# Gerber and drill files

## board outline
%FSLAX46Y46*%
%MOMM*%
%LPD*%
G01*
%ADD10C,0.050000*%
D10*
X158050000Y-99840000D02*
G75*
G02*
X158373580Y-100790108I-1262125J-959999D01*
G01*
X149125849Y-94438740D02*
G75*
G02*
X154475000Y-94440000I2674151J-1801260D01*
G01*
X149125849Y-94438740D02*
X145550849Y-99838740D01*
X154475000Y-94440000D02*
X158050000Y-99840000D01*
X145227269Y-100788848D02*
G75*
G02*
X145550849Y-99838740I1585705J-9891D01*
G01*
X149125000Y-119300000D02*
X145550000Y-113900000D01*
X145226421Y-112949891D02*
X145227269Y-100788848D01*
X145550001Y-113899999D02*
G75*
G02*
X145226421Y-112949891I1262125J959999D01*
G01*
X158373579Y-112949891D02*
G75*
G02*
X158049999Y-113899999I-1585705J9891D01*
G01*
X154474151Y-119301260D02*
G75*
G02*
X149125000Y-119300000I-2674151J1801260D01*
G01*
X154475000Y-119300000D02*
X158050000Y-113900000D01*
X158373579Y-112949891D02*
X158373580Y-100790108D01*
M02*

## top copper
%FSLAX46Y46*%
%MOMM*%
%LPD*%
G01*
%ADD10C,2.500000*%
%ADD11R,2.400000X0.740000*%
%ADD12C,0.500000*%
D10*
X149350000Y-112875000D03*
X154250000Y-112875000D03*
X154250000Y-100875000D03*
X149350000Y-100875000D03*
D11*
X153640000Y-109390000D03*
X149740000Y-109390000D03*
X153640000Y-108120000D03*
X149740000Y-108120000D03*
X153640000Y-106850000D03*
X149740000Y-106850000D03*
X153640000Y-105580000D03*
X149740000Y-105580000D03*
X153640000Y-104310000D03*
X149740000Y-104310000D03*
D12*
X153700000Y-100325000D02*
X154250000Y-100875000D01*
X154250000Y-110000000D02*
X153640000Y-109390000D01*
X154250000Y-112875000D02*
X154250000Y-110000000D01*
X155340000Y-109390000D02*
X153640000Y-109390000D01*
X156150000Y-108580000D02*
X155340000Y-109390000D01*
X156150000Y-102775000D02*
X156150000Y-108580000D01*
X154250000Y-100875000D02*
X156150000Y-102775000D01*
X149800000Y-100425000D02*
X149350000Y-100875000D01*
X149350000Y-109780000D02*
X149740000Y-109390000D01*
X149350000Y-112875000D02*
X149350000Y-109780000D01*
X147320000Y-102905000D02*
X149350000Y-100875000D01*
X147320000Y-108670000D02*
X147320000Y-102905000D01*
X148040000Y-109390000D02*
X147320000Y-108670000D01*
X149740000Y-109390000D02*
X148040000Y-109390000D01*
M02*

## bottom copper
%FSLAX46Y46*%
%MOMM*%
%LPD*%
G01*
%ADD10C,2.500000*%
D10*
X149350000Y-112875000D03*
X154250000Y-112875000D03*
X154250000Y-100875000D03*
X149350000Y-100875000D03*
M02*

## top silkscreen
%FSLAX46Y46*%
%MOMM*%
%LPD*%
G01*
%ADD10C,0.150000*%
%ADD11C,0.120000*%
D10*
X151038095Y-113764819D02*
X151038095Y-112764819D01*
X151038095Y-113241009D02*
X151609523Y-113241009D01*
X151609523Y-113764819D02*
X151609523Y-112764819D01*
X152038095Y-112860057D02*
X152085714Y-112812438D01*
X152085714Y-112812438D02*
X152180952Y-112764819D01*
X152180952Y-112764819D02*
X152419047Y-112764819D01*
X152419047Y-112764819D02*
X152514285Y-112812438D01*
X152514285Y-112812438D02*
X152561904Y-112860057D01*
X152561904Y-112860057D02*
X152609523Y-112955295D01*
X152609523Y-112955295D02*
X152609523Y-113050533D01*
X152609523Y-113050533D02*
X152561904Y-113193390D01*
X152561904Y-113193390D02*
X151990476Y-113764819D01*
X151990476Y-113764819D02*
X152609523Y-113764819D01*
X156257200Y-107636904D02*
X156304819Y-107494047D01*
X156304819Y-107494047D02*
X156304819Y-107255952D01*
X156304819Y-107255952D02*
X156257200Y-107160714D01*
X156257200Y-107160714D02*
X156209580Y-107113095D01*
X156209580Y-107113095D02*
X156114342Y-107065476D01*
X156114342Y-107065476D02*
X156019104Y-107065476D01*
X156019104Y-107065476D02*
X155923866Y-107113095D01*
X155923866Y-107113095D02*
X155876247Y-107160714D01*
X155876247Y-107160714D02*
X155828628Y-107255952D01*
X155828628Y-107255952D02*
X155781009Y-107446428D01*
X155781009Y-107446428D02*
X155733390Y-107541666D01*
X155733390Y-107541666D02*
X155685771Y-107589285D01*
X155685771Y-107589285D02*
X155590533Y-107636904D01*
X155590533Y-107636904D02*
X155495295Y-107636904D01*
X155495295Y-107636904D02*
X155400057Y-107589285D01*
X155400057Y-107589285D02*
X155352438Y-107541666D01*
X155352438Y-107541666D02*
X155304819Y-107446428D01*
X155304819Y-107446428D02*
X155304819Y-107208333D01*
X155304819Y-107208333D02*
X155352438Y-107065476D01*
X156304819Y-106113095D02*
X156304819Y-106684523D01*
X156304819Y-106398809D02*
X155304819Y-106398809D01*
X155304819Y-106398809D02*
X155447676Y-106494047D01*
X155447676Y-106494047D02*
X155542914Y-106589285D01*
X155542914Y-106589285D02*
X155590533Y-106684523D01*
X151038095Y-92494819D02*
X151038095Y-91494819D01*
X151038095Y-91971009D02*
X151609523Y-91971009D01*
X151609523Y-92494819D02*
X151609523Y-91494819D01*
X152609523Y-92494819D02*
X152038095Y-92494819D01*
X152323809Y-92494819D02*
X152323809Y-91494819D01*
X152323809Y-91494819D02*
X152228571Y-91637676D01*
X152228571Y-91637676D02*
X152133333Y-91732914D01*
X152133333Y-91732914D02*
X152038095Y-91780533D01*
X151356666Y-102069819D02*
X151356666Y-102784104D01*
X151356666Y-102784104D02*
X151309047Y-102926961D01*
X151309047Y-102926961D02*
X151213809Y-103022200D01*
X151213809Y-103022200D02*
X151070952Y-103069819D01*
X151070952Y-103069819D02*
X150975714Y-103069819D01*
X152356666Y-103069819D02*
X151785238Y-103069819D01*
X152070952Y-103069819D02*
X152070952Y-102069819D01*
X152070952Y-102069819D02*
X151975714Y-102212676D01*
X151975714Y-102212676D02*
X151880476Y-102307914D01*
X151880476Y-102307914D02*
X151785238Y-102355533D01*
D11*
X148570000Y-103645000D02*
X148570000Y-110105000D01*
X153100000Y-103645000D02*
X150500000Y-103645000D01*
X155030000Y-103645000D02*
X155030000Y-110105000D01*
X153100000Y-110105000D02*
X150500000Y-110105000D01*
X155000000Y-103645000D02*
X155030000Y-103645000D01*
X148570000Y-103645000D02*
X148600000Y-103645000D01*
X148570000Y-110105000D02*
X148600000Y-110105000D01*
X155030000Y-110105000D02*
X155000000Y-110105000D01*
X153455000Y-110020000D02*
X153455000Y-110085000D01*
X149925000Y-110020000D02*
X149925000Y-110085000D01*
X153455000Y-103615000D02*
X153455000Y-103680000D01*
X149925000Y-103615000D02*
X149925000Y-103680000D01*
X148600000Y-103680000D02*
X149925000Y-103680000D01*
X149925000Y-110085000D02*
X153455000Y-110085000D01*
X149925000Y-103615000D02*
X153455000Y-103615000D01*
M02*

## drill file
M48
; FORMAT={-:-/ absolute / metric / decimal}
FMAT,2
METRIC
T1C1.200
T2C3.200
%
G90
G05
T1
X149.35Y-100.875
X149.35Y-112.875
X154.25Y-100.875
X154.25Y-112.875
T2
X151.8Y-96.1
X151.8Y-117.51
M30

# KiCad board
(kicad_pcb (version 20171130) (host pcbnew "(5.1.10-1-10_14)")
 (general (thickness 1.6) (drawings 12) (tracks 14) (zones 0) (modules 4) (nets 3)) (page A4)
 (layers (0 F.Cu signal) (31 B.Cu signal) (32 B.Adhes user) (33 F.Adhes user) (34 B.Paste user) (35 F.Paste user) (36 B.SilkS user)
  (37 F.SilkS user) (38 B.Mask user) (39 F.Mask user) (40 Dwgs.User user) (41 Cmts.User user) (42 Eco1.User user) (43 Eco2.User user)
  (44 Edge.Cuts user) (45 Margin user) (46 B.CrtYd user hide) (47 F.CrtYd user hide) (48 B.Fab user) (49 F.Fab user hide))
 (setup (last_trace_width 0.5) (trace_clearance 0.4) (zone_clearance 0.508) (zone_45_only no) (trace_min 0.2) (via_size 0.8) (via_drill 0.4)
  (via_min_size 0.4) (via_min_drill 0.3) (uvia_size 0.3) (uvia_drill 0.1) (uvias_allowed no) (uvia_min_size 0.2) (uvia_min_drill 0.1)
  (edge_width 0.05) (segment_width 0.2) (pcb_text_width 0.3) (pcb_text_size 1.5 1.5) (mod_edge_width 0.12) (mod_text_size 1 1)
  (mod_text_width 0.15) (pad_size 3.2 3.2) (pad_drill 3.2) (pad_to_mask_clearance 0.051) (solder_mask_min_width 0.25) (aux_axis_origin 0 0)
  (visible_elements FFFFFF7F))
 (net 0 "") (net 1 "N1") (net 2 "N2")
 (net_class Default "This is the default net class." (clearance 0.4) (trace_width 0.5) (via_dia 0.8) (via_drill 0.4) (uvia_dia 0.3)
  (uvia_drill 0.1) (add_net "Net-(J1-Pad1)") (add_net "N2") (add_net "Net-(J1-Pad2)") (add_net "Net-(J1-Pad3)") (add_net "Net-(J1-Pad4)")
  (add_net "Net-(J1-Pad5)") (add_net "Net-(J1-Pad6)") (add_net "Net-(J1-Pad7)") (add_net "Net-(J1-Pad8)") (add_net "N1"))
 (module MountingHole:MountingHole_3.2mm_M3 (layer F.Cu) (at 151.8 117.51)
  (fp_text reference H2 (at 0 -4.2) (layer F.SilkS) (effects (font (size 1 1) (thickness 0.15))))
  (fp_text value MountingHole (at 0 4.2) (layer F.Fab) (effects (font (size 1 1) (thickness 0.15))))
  (pad 1 np_thru_hole circle (at 0 0) (size 3.2 3.2) (drill 3.2) (layers *.Cu *.Mask)))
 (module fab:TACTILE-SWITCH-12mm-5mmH (layer F.Cu) (at 151.8 106.875 270)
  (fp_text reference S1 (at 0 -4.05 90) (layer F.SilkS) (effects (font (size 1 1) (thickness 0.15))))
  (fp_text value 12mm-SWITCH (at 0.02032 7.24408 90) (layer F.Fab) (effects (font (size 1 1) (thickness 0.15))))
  (fp_line (start -3.23 3.23) (end 3.23 3.23) (layer F.SilkS) (width 0.12))
  (fp_line (start -3.23 -1.3) (end -3.23 1.3) (layer F.SilkS) (width 0.12))
  (fp_line (start -3.23 -3.23) (end 3.23 -3.23) (layer F.SilkS) (width 0.12))
  (fp_line (start 3.23 -1.3) (end 3.23 1.3) (layer F.SilkS) (width 0.12))
  (fp_line (start -3.23 -3.2) (end -3.23 -3.23) (layer F.SilkS) (width 0.12))
  (fp_line (start -3.23 3.23) (end -3.23 3.2) (layer F.SilkS) (width 0.12))
  (fp_line (start 3.23 3.23) (end 3.23 3.2) (layer F.SilkS) (width 0.12))
  (fp_line (start 3.23 -3.23) (end 3.23 -3.2) (layer F.SilkS) (width 0.12))
  (pad 4 thru_hole circle (at 6 2.45 270) (size 2.5 2.5) (drill 1.2) (layers *.Cu *.Mask) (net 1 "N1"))
  (pad 2 thru_hole circle (at 6 -2.45 270) (size 2.5 2.5) (drill 1.2) (layers *.Cu *.Mask) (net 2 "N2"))
  (pad 1 thru_hole circle (at -6 -2.45 270) (size 2.5 2.5) (drill 1.2) (layers *.Cu *.Mask) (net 2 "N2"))
  (pad 3 thru_hole circle (at -6 2.45 270) (size 2.5 2.5) (drill 1.2) (layers *.Cu *.Mask) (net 1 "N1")))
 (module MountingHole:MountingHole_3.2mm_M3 (layer F.Cu) (at 151.8 96.24)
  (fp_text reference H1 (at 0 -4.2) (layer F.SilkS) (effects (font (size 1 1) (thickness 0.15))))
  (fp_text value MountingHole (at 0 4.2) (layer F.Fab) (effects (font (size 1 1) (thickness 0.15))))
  (pad "" np_thru_hole circle (at 0 -0.14) (size 3.2 3.2) (drill 3.2) (layers *.Cu *.Mask)))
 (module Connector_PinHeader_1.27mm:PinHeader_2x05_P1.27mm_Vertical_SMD (layer F.Cu) (at 151.69 106.85)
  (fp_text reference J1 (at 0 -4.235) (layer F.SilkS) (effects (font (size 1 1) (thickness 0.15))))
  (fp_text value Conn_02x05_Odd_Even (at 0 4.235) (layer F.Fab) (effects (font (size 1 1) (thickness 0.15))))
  (fp_line (start 1.765 3.17) (end 1.765 3.235) (layer F.SilkS) (width 0.12))
  (fp_line (start -1.765 3.17) (end -1.765 3.235) (layer F.SilkS) (width 0.12))
  (fp_line (start 1.765 -3.235) (end 1.765 -3.17) (layer F.SilkS) (width 0.12))
  (fp_line (start -1.765 -3.235) (end -1.765 -3.17) (layer F.SilkS) (width 0.12))
  (fp_line (start -3.09 -3.17) (end -1.765 -3.17) (layer F.SilkS) (width 0.12))
  (fp_line (start -1.765 3.235) (end 1.765 3.235) (layer F.SilkS) (width 0.12))
  (fp_line (start -1.765 -3.235) (end 1.765 -3.235) (layer F.SilkS) (width 0.12))
  (pad 10 smd rect (at 1.95 2.54) (size 2.4 0.74) (layers F.Cu F.Paste F.Mask) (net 2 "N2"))
  (pad 9 smd rect (at -1.95 2.54) (size 2.4 0.74) (layers F.Cu F.Paste F.Mask) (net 1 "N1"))
  (pad 8 smd rect (at 1.95 1.27) (size 2.4 0.74) (layers F.Cu F.Paste F.Mask))
  (pad 7 smd rect (at -1.95 1.27) (size 2.4 0.74) (layers F.Cu F.Paste F.Mask))
  (pad 6 smd rect (at 1.95 0) (size 2.4 0.74) (layers F.Cu F.Paste F.Mask))
  (pad 5 smd rect (at -1.95 0) (size 2.4 0.74) (layers F.Cu F.Paste F.Mask))
  (pad 4 smd rect (at 1.95 -1.27) (size 2.4 0.74) (layers F.Cu F.Paste F.Mask))
  (pad 3 smd rect (at -1.95 -1.27) (size 2.4 0.74) (layers F.Cu F.Paste F.Mask))
  (pad 2 smd rect (at 1.95 -2.54) (size 2.4 0.74) (layers F.Cu F.Paste F.Mask))
  (pad 1 smd rect (at -1.95 -2.54) (size 2.4 0.74) (layers F.Cu F.Paste F.Mask)))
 (gr_arc (start 156.787875 100.799999) (end 158.05 99.84) (angle 36.9) (layer Edge.Cuts) (width 0.05))
 (gr_arc (start 151.8 96.24) (end 154.475 94.44) (angle -112.1) (layer Edge.Cuts) (width 0.05))
 (gr_line (start 149.125849 94.43874) (end 145.550849 99.83874) (layer Edge.Cuts) (width 0.05))
 (gr_line (start 154.475 94.44) (end 158.05 99.84) (layer Edge.Cuts) (width 0.05))
 (gr_arc (start 146.812974 100.798739) (end 145.550849 99.83874) (angle -36.9) (layer Edge.Cuts) (width 0.05))
 (gr_line (start 149.125 119.3) (end 145.55 113.9) (layer Edge.Cuts) (width 0.05))
 (gr_line (start 145.226421 112.949891) (end 145.227269 100.788848) (layer Edge.Cuts) (width 0.05))
 (gr_arc (start 146.812126 112.94) (end 145.550001 113.899999) (angle 36.9) (layer Edge.Cuts) (width 0.05))
 (gr_arc (start 156.787874 112.94) (end 158.049999 113.899999) (angle -36.9) (layer Edge.Cuts) (width 0.05))
 (gr_arc (start 151.8 117.5) (end 149.125 119.3) (angle -112.1) (layer Edge.Cuts) (width 0.05))
 (gr_line (start 154.475 119.3) (end 158.05 113.9) (layer Edge.Cuts) (width 0.05))
 (gr_line (start 158.373579 112.949891) (end 158.37358 100.790108) (layer Edge.Cuts) (width 0.05))
 (segment (start 153.7 100.325) (end 154.25 100.875) (width 0.5) (layer F.Cu) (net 2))
 (segment (start 154.25 110) (end 153.64 109.39) (width 0.5) (layer F.Cu) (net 2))
 (segment (start 154.25 112.875) (end 154.25 110) (width 0.5) (layer F.Cu) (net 2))
 (segment (start 155.34 109.39) (end 153.64 109.39) (width 0.5) (layer F.Cu) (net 2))
 (segment (start 156.15 108.58) (end 155.34 109.39) (width 0.5) (layer F.Cu) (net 2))
 (segment (start 156.15 102.775) (end 156.15 108.58) (width 0.5) (layer F.Cu) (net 2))
 (segment (start 154.25 100.875) (end 156.15 102.775) (width 0.5) (layer F.Cu) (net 2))
 (segment (start 149.8 100.425) (end 149.35 100.875) (width 0.5) (layer F.Cu) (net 1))
 (segment (start 149.35 109.78) (end 149.74 109.39) (width 0.5) (layer F.Cu) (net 1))
 (segment (start 149.35 112.875) (end 149.35 109.78) (width 0.5) (layer F.Cu) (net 1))
 (segment (start 147.32 102.905) (end 149.35 100.875) (width 0.5) (layer F.Cu) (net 1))
 (segment (start 147.32 108.67) (end 147.32 102.905) (width 0.5) (layer F.Cu) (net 1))
 (segment (start 148.04 109.39) (end 147.32 108.67) (width 0.5) (layer F.Cu) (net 1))
 (segment (start 149.74 109.39) (end 148.04 109.39) (width 0.5) (layer F.Cu) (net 1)))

